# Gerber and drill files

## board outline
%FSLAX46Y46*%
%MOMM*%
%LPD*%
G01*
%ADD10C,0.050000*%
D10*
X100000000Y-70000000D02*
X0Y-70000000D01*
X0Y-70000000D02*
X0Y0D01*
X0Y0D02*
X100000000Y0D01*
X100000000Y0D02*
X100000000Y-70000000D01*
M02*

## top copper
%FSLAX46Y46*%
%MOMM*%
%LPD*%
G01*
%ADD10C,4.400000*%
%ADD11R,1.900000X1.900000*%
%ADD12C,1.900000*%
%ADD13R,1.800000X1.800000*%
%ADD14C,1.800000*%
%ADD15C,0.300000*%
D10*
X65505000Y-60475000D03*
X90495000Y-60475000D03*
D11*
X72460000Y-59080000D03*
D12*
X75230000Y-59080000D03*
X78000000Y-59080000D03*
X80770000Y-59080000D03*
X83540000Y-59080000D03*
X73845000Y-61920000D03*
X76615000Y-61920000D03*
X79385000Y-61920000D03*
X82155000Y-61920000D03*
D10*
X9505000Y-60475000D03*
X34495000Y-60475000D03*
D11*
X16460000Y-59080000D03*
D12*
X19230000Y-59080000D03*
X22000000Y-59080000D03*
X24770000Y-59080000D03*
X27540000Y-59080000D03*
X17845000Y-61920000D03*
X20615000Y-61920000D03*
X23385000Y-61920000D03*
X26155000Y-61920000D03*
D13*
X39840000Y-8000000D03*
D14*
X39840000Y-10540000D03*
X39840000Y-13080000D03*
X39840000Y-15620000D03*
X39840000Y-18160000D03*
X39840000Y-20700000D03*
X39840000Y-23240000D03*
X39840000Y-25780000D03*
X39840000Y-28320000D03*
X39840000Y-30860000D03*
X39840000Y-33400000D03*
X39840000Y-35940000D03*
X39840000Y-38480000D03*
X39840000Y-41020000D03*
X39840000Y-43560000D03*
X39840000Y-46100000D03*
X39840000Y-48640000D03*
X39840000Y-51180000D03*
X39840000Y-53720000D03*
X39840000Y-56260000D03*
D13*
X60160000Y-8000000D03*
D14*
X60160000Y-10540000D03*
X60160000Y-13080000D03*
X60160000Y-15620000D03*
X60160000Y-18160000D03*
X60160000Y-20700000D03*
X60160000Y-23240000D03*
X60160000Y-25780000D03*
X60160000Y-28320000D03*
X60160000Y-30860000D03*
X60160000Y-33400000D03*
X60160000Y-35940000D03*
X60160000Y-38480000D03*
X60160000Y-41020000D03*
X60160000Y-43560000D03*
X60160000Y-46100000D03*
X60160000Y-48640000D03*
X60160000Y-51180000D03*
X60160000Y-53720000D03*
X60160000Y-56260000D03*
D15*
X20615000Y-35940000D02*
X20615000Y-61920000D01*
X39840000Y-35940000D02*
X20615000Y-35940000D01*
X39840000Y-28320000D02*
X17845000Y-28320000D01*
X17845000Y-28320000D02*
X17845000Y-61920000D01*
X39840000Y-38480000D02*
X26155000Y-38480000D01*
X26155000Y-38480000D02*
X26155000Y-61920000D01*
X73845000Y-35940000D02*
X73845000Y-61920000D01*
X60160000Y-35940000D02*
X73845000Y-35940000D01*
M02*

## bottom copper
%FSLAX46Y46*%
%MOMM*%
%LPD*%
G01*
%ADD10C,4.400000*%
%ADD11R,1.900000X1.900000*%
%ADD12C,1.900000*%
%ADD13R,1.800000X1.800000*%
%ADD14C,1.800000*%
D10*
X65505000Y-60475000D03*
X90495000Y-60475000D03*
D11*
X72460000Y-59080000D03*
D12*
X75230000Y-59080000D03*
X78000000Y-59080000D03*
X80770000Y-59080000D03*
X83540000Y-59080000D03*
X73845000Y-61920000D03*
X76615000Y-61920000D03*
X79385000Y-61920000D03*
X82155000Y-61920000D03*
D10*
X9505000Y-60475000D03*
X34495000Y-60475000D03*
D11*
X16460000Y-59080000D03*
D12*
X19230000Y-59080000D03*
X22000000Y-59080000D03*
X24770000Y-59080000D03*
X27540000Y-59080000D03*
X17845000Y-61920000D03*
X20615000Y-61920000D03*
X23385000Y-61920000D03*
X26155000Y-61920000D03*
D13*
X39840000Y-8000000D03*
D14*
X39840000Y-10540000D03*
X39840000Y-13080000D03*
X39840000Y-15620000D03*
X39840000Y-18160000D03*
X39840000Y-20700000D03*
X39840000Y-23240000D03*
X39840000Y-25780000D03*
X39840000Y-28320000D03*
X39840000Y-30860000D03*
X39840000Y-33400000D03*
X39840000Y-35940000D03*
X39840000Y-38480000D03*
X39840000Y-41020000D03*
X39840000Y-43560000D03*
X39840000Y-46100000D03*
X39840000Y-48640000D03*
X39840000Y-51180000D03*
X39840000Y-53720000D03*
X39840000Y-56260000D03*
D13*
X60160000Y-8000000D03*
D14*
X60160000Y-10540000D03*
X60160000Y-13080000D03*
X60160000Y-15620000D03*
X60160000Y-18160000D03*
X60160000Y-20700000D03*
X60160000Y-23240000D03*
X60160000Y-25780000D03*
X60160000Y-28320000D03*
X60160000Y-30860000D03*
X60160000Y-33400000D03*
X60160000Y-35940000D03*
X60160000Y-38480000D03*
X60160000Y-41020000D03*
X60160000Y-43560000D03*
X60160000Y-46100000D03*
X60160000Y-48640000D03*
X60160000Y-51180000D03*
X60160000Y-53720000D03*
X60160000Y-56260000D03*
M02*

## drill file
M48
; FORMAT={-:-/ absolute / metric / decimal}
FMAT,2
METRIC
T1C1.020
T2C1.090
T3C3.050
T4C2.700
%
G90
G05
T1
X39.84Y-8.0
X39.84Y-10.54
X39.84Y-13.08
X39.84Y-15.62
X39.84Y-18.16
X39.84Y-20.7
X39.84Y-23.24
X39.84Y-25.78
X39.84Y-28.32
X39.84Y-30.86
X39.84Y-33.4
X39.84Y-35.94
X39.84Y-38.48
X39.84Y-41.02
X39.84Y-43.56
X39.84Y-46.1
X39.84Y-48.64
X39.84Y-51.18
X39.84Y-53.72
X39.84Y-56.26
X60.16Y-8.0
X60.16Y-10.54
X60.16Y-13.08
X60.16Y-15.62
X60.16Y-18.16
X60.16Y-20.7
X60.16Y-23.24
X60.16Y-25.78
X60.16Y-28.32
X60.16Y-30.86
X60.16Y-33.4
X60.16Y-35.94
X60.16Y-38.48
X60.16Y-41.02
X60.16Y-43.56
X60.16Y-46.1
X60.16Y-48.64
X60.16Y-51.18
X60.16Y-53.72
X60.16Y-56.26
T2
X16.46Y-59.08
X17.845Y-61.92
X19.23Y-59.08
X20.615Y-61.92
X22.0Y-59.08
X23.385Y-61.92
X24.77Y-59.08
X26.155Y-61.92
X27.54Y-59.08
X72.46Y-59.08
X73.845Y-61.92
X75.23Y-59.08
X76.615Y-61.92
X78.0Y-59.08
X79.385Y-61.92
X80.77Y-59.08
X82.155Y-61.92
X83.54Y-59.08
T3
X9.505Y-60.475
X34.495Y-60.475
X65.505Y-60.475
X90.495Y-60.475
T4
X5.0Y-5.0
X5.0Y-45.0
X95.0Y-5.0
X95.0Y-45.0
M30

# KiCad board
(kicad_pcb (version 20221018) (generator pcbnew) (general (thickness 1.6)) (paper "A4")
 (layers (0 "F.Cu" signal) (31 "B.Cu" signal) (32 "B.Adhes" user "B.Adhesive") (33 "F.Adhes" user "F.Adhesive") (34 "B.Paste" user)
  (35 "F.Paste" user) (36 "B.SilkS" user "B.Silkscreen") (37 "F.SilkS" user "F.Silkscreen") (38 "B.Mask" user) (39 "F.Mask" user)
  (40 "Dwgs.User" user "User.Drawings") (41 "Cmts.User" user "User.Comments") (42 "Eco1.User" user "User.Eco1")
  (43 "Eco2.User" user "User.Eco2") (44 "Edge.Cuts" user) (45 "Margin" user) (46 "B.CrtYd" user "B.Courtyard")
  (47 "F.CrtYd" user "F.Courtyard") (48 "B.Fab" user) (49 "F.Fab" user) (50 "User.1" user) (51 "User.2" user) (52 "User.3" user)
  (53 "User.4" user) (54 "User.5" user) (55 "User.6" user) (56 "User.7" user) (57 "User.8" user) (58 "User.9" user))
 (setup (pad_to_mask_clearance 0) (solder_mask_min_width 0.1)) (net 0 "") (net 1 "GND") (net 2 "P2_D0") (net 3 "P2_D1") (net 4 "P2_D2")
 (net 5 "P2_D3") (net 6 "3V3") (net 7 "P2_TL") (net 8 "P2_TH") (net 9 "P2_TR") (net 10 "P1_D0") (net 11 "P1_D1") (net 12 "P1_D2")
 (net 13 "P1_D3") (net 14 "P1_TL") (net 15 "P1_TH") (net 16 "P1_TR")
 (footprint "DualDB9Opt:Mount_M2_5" (layer "F.Cu") (at 5 45)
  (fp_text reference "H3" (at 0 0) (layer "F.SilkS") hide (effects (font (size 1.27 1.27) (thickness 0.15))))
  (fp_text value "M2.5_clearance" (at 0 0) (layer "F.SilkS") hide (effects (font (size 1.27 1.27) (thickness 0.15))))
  (pad "" np_thru_hole circle (at 0 0) (size 2.7 2.7) (drill 2.7) (layers "F&B.Cu" "*.Mask")))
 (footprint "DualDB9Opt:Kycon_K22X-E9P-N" (layer "F.Cu") (at 72.46 59.08)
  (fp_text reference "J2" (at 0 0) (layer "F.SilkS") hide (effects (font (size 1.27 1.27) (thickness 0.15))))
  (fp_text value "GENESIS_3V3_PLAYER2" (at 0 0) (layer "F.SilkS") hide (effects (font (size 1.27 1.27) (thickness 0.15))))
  (pad "0" thru_hole circle (at -6.955 1.395) (size 4.4 4.4) (drill 3.05) (layers "F&B.Cu" "*.Mask") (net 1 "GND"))
  (pad "0" thru_hole circle (at 18.035 1.395) (size 4.4 4.4) (drill 3.05) (layers "F&B.Cu" "*.Mask") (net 1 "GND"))
  (pad "1" thru_hole rect (at 0 0) (size 1.9 1.9) (drill 1.09) (layers "F&B.Cu" "*.Mask") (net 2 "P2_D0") (thermal_bridge_angle 45))
  (pad "2" thru_hole circle (at 2.77 0) (size 1.9 1.9) (drill 1.09) (layers "F&B.Cu" "*.Mask") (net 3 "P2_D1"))
  (pad "3" thru_hole circle (at 5.54 0) (size 1.9 1.9) (drill 1.09) (layers "F&B.Cu" "*.Mask") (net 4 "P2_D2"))
  (pad "4" thru_hole circle (at 8.31 0) (size 1.9 1.9) (drill 1.09) (layers "F&B.Cu" "*.Mask") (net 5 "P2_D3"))
  (pad "5" thru_hole circle (at 11.08 0) (size 1.9 1.9) (drill 1.09) (layers "F&B.Cu" "*.Mask") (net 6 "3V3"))
  (pad "6" thru_hole circle (at 1.385 2.84) (size 1.9 1.9) (drill 1.09) (layers "F&B.Cu" "*.Mask") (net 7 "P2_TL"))
  (pad "7" thru_hole circle (at 4.155 2.84) (size 1.9 1.9) (drill 1.09) (layers "F&B.Cu" "*.Mask") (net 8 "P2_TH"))
  (pad "8" thru_hole circle (at 6.925 2.84) (size 1.9 1.9) (drill 1.09) (layers "F&B.Cu" "*.Mask") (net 1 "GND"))
  (pad "9" thru_hole circle (at 9.695 2.84) (size 1.9 1.9) (drill 1.09) (layers "F&B.Cu" "*.Mask") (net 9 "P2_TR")))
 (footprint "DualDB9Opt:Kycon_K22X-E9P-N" (layer "F.Cu") (at 16.46 59.08)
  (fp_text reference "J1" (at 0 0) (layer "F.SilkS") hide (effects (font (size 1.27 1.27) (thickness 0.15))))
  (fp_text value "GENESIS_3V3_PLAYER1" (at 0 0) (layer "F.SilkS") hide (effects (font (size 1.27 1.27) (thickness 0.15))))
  (pad "0" thru_hole circle (at -6.955 1.395) (size 4.4 4.4) (drill 3.05) (layers "F&B.Cu" "*.Mask") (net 1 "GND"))
  (pad "0" thru_hole circle (at 18.035 1.395) (size 4.4 4.4) (drill 3.05) (layers "F&B.Cu" "*.Mask") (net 1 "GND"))
  (pad "1" thru_hole rect (at 0 0) (size 1.9 1.9) (drill 1.09) (layers "F&B.Cu" "*.Mask") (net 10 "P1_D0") (thermal_bridge_angle 45))
  (pad "2" thru_hole circle (at 2.77 0) (size 1.9 1.9) (drill 1.09) (layers "F&B.Cu" "*.Mask") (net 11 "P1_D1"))
  (pad "3" thru_hole circle (at 5.54 0) (size 1.9 1.9) (drill 1.09) (layers "F&B.Cu" "*.Mask") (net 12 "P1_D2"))
  (pad "4" thru_hole circle (at 8.31 0) (size 1.9 1.9) (drill 1.09) (layers "F&B.Cu" "*.Mask") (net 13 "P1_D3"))
  (pad "5" thru_hole circle (at 11.08 0) (size 1.9 1.9) (drill 1.09) (layers "F&B.Cu" "*.Mask") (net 6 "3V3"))
  (pad "6" thru_hole circle (at 1.385 2.84) (size 1.9 1.9) (drill 1.09) (layers "F&B.Cu" "*.Mask") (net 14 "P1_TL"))
  (pad "7" thru_hole circle (at 4.155 2.84) (size 1.9 1.9) (drill 1.09) (layers "F&B.Cu" "*.Mask") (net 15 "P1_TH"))
  (pad "8" thru_hole circle (at 6.925 2.84) (size 1.9 1.9) (drill 1.09) (layers "F&B.Cu" "*.Mask") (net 1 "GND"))
  (pad "9" thru_hole circle (at 9.695 2.84) (size 1.9 1.9) (drill 1.09) (layers "F&B.Cu" "*.Mask") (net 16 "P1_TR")))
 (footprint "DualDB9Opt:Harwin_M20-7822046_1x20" (layer "F.Cu") (at 39.84 8)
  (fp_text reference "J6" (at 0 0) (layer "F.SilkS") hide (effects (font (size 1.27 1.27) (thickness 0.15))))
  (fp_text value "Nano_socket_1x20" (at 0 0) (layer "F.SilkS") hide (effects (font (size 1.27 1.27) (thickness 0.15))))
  (pad "1" thru_hole rect (at 0 0) (size 1.8 1.8) (drill 1.02) (layers "F&B.Cu" "*.Mask") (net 10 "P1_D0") (thermal_bridge_angle 45))
  (pad "2" thru_hole circle (at 0 2.54) (size 1.8 1.8) (drill 1.02) (layers "F&B.Cu" "*.Mask") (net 11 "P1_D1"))
  (pad "3" thru_hole circle (at 0 5.08) (size 1.8 1.8) (drill 1.02) (layers "F&B.Cu" "*.Mask"))
  (pad "4" thru_hole circle (at 0 7.62) (size 1.8 1.8) (drill 1.02) (layers "F&B.Cu" "*.Mask"))
  (pad "5" thru_hole circle (at 0 10.16) (size 1.8 1.8) (drill 1.02) (layers "F&B.Cu" "*.Mask") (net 12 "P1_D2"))
  (pad "6" thru_hole circle (at 0 12.7) (size 1.8 1.8) (drill 1.02) (layers "F&B.Cu" "*.Mask"))
  (pad "7" thru_hole circle (at 0 15.24) (size 1.8 1.8) (drill 1.02) (layers "F&B.Cu" "*.Mask"))
  (pad "8" thru_hole circle (at 0 17.78) (size 1.8 1.8) (drill 1.02) (layers "F&B.Cu" "*.Mask") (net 13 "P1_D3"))
  (pad "9" thru_hole circle (at 0 20.32) (size 1.8 1.8) (drill 1.02) (layers "F&B.Cu" "*.Mask") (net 14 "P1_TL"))
  (pad "10" thru_hole circle (at 0 22.86) (size 1.8 1.8) (drill 1.02) (layers "F&B.Cu" "*.Mask"))
  (pad "11" thru_hole circle (at 0 25.4) (size 1.8 1.8) (drill 1.02) (layers "F&B.Cu" "*.Mask"))
  (pad "12" thru_hole circle (at 0 27.94) (size 1.8 1.8) (drill 1.02) (layers "F&B.Cu" "*.Mask") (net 15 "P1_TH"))
  (pad "13" thru_hole circle (at 0 30.48) (size 1.8 1.8) (drill 1.02) (layers "F&B.Cu" "*.Mask") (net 16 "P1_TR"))
  (pad "14" thru_hole circle (at 0 33.02) (size 1.8 1.8) (drill 1.02) (layers "F&B.Cu" "*.Mask"))
  (pad "15" thru_hole circle (at 0 35.56) (size 1.8 1.8) (drill 1.02) (layers "F&B.Cu" "*.Mask"))
  (pad "16" thru_hole circle (at 0 38.1) (size 1.8 1.8) (drill 1.02) (layers "F&B.Cu" "*.Mask"))
  (pad "17" thru_hole circle (at 0 40.64) (size 1.8 1.8) (drill 1.02) (layers "F&B.Cu" "*.Mask"))
  (pad "18" thru_hole circle (at 0 43.18) (size 1.8 1.8) (drill 1.02) (layers "F&B.Cu" "*.Mask"))
  (pad "19" thru_hole circle (at 0 45.72) (size 1.8 1.8) (drill 1.02) (layers "F&B.Cu" "*.Mask") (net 6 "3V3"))
  (pad "20" thru_hole circle (at 0 48.26) (size 1.8 1.8) (drill 1.02) (layers "F&B.Cu" "*.Mask") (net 1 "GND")))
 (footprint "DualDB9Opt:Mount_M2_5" (layer "F.Cu") (at 95 45)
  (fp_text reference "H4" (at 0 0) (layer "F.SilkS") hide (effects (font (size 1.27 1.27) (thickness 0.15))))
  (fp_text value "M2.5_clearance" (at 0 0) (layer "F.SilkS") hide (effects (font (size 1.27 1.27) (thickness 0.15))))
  (pad "" np_thru_hole circle (at 0 0) (size 2.7 2.7) (drill 2.7) (layers "F&B.Cu" "*.Mask")))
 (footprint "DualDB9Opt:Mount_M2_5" (layer "F.Cu") (at 95 5)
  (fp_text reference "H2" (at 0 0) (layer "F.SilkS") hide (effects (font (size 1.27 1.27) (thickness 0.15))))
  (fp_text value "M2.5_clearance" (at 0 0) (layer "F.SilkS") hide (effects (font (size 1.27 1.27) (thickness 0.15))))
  (pad "" np_thru_hole circle (at 0 0) (size 2.7 2.7) (drill 2.7) (layers "F&B.Cu" "*.Mask")))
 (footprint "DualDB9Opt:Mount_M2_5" (layer "F.Cu") (at 5 5)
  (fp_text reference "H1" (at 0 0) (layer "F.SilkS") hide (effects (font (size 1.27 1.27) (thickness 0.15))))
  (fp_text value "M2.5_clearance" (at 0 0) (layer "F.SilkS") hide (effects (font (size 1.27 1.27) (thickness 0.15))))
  (pad "" np_thru_hole circle (at 0 0) (size 2.7 2.7) (drill 2.7) (layers "F&B.Cu" "*.Mask")))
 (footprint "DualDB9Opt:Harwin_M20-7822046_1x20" (layer "F.Cu") (at 60.16 8)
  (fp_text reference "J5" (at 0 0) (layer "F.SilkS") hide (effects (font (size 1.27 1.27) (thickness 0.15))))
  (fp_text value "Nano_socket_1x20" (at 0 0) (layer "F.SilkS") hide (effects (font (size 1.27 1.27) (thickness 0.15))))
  (pad "1" thru_hole rect (at 0 0) (size 1.8 1.8) (drill 1.02) (layers "F&B.Cu" "*.Mask") (thermal_bridge_angle 45))
  (pad "2" thru_hole circle (at 0 2.54) (size 1.8 1.8) (drill 1.02) (layers "F&B.Cu" "*.Mask"))
  (pad "3" thru_hole circle (at 0 5.08) (size 1.8 1.8) (drill 1.02) (layers "F&B.Cu" "*.Mask"))
  (pad "4" thru_hole circle (at 0 7.62) (size 1.8 1.8) (drill 1.02) (layers "F&B.Cu" "*.Mask"))
  (pad "5" thru_hole circle (at 0 10.16) (size 1.8 1.8) (drill 1.02) (layers "F&B.Cu" "*.Mask") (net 2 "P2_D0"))
  (pad "6" thru_hole circle (at 0 12.7) (size 1.8 1.8) (drill 1.02) (layers "F&B.Cu" "*.Mask") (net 3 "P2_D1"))
  (pad "7" thru_hole circle (at 0 15.24) (size 1.8 1.8) (drill 1.02) (layers "F&B.Cu" "*.Mask"))
  (pad "8" thru_hole circle (at 0 17.78) (size 1.8 1.8) (drill 1.02) (layers "F&B.Cu" "*.Mask"))
  (pad "9" thru_hole circle (at 0 20.32) (size 1.8 1.8) (drill 1.02) (layers "F&B.Cu" "*.Mask") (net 4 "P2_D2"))
  (pad "10" thru_hole circle (at 0 22.86) (size 1.8 1.8) (drill 1.02) (layers "F&B.Cu" "*.Mask") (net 5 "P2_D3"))
  (pad "11" thru_hole circle (at 0 25.4) (size 1.8 1.8) (drill 1.02) (layers "F&B.Cu" "*.Mask"))
  (pad "12" thru_hole circle (at 0 27.94) (size 1.8 1.8) (drill 1.02) (layers "F&B.Cu" "*.Mask") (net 7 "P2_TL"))
  (pad "13" thru_hole circle (at 0 30.48) (size 1.8 1.8) (drill 1.02) (layers "F&B.Cu" "*.Mask"))
  (pad "14" thru_hole circle (at 0 33.02) (size 1.8 1.8) (drill 1.02) (layers "F&B.Cu" "*.Mask"))
  (pad "15" thru_hole circle (at 0 35.56) (size 1.8 1.8) (drill 1.02) (layers "F&B.Cu" "*.Mask") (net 1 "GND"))
  (pad "16" thru_hole circle (at 0 38.1) (size 1.8 1.8) (drill 1.02) (layers "F&B.Cu" "*.Mask") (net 6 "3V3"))
  (pad "17" thru_hole circle (at 0 40.64) (size 1.8 1.8) (drill 1.02) (layers "F&B.Cu" "*.Mask") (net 8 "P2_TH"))
  (pad "18" thru_hole circle (at 0 43.18) (size 1.8 1.8) (drill 1.02) (layers "F&B.Cu" "*.Mask") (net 9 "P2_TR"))
  (pad "19" thru_hole circle (at 0 45.72) (size 1.8 1.8) (drill 1.02) (layers "F&B.Cu" "*.Mask"))
  (pad "20" thru_hole circle (at 0 48.26) (size 1.8 1.8) (drill 1.02) (layers "F&B.Cu" "*.Mask")))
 (gr_line (start 100 70) (end 0 70) (stroke (width 0.05) (type default)) (layer "Edge.Cuts"))
 (gr_line (start 0 70) (end 0 0) (stroke (width 0.05) (type default)) (layer "Edge.Cuts"))
 (gr_line (start 0 0) (end 100 0) (stroke (width 0.05) (type default)) (layer "Edge.Cuts"))
 (gr_line (start 100 0) (end 100 70) (stroke (width 0.05) (type default)) (layer "Edge.Cuts"))
 (segment (start 20.615 35.94) (end 20.615 61.92) (width 0.3) (layer "F.Cu") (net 15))
 (segment (start 39.84 35.94) (end 20.615 35.94) (width 0.3) (layer "F.Cu") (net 15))
 (segment (start 39.84 28.32) (end 17.845 28.32) (width 0.3) (layer "F.Cu") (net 14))
 (segment (start 17.845 28.32) (end 17.845 61.92) (width 0.3) (layer "F.Cu") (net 14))
 (segment (start 39.84 38.48) (end 26.155 38.48) (width 0.3) (layer "F.Cu") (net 16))
 (segment (start 26.155 38.48) (end 26.155 61.92) (width 0.3) (layer "F.Cu") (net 16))
 (segment (start 73.845 35.94) (end 73.845 61.92) (width 0.3) (layer "F.Cu") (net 7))
 (segment (start 60.16 35.94) (end 73.845 35.94) (width 0.3) (layer "F.Cu") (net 7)))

